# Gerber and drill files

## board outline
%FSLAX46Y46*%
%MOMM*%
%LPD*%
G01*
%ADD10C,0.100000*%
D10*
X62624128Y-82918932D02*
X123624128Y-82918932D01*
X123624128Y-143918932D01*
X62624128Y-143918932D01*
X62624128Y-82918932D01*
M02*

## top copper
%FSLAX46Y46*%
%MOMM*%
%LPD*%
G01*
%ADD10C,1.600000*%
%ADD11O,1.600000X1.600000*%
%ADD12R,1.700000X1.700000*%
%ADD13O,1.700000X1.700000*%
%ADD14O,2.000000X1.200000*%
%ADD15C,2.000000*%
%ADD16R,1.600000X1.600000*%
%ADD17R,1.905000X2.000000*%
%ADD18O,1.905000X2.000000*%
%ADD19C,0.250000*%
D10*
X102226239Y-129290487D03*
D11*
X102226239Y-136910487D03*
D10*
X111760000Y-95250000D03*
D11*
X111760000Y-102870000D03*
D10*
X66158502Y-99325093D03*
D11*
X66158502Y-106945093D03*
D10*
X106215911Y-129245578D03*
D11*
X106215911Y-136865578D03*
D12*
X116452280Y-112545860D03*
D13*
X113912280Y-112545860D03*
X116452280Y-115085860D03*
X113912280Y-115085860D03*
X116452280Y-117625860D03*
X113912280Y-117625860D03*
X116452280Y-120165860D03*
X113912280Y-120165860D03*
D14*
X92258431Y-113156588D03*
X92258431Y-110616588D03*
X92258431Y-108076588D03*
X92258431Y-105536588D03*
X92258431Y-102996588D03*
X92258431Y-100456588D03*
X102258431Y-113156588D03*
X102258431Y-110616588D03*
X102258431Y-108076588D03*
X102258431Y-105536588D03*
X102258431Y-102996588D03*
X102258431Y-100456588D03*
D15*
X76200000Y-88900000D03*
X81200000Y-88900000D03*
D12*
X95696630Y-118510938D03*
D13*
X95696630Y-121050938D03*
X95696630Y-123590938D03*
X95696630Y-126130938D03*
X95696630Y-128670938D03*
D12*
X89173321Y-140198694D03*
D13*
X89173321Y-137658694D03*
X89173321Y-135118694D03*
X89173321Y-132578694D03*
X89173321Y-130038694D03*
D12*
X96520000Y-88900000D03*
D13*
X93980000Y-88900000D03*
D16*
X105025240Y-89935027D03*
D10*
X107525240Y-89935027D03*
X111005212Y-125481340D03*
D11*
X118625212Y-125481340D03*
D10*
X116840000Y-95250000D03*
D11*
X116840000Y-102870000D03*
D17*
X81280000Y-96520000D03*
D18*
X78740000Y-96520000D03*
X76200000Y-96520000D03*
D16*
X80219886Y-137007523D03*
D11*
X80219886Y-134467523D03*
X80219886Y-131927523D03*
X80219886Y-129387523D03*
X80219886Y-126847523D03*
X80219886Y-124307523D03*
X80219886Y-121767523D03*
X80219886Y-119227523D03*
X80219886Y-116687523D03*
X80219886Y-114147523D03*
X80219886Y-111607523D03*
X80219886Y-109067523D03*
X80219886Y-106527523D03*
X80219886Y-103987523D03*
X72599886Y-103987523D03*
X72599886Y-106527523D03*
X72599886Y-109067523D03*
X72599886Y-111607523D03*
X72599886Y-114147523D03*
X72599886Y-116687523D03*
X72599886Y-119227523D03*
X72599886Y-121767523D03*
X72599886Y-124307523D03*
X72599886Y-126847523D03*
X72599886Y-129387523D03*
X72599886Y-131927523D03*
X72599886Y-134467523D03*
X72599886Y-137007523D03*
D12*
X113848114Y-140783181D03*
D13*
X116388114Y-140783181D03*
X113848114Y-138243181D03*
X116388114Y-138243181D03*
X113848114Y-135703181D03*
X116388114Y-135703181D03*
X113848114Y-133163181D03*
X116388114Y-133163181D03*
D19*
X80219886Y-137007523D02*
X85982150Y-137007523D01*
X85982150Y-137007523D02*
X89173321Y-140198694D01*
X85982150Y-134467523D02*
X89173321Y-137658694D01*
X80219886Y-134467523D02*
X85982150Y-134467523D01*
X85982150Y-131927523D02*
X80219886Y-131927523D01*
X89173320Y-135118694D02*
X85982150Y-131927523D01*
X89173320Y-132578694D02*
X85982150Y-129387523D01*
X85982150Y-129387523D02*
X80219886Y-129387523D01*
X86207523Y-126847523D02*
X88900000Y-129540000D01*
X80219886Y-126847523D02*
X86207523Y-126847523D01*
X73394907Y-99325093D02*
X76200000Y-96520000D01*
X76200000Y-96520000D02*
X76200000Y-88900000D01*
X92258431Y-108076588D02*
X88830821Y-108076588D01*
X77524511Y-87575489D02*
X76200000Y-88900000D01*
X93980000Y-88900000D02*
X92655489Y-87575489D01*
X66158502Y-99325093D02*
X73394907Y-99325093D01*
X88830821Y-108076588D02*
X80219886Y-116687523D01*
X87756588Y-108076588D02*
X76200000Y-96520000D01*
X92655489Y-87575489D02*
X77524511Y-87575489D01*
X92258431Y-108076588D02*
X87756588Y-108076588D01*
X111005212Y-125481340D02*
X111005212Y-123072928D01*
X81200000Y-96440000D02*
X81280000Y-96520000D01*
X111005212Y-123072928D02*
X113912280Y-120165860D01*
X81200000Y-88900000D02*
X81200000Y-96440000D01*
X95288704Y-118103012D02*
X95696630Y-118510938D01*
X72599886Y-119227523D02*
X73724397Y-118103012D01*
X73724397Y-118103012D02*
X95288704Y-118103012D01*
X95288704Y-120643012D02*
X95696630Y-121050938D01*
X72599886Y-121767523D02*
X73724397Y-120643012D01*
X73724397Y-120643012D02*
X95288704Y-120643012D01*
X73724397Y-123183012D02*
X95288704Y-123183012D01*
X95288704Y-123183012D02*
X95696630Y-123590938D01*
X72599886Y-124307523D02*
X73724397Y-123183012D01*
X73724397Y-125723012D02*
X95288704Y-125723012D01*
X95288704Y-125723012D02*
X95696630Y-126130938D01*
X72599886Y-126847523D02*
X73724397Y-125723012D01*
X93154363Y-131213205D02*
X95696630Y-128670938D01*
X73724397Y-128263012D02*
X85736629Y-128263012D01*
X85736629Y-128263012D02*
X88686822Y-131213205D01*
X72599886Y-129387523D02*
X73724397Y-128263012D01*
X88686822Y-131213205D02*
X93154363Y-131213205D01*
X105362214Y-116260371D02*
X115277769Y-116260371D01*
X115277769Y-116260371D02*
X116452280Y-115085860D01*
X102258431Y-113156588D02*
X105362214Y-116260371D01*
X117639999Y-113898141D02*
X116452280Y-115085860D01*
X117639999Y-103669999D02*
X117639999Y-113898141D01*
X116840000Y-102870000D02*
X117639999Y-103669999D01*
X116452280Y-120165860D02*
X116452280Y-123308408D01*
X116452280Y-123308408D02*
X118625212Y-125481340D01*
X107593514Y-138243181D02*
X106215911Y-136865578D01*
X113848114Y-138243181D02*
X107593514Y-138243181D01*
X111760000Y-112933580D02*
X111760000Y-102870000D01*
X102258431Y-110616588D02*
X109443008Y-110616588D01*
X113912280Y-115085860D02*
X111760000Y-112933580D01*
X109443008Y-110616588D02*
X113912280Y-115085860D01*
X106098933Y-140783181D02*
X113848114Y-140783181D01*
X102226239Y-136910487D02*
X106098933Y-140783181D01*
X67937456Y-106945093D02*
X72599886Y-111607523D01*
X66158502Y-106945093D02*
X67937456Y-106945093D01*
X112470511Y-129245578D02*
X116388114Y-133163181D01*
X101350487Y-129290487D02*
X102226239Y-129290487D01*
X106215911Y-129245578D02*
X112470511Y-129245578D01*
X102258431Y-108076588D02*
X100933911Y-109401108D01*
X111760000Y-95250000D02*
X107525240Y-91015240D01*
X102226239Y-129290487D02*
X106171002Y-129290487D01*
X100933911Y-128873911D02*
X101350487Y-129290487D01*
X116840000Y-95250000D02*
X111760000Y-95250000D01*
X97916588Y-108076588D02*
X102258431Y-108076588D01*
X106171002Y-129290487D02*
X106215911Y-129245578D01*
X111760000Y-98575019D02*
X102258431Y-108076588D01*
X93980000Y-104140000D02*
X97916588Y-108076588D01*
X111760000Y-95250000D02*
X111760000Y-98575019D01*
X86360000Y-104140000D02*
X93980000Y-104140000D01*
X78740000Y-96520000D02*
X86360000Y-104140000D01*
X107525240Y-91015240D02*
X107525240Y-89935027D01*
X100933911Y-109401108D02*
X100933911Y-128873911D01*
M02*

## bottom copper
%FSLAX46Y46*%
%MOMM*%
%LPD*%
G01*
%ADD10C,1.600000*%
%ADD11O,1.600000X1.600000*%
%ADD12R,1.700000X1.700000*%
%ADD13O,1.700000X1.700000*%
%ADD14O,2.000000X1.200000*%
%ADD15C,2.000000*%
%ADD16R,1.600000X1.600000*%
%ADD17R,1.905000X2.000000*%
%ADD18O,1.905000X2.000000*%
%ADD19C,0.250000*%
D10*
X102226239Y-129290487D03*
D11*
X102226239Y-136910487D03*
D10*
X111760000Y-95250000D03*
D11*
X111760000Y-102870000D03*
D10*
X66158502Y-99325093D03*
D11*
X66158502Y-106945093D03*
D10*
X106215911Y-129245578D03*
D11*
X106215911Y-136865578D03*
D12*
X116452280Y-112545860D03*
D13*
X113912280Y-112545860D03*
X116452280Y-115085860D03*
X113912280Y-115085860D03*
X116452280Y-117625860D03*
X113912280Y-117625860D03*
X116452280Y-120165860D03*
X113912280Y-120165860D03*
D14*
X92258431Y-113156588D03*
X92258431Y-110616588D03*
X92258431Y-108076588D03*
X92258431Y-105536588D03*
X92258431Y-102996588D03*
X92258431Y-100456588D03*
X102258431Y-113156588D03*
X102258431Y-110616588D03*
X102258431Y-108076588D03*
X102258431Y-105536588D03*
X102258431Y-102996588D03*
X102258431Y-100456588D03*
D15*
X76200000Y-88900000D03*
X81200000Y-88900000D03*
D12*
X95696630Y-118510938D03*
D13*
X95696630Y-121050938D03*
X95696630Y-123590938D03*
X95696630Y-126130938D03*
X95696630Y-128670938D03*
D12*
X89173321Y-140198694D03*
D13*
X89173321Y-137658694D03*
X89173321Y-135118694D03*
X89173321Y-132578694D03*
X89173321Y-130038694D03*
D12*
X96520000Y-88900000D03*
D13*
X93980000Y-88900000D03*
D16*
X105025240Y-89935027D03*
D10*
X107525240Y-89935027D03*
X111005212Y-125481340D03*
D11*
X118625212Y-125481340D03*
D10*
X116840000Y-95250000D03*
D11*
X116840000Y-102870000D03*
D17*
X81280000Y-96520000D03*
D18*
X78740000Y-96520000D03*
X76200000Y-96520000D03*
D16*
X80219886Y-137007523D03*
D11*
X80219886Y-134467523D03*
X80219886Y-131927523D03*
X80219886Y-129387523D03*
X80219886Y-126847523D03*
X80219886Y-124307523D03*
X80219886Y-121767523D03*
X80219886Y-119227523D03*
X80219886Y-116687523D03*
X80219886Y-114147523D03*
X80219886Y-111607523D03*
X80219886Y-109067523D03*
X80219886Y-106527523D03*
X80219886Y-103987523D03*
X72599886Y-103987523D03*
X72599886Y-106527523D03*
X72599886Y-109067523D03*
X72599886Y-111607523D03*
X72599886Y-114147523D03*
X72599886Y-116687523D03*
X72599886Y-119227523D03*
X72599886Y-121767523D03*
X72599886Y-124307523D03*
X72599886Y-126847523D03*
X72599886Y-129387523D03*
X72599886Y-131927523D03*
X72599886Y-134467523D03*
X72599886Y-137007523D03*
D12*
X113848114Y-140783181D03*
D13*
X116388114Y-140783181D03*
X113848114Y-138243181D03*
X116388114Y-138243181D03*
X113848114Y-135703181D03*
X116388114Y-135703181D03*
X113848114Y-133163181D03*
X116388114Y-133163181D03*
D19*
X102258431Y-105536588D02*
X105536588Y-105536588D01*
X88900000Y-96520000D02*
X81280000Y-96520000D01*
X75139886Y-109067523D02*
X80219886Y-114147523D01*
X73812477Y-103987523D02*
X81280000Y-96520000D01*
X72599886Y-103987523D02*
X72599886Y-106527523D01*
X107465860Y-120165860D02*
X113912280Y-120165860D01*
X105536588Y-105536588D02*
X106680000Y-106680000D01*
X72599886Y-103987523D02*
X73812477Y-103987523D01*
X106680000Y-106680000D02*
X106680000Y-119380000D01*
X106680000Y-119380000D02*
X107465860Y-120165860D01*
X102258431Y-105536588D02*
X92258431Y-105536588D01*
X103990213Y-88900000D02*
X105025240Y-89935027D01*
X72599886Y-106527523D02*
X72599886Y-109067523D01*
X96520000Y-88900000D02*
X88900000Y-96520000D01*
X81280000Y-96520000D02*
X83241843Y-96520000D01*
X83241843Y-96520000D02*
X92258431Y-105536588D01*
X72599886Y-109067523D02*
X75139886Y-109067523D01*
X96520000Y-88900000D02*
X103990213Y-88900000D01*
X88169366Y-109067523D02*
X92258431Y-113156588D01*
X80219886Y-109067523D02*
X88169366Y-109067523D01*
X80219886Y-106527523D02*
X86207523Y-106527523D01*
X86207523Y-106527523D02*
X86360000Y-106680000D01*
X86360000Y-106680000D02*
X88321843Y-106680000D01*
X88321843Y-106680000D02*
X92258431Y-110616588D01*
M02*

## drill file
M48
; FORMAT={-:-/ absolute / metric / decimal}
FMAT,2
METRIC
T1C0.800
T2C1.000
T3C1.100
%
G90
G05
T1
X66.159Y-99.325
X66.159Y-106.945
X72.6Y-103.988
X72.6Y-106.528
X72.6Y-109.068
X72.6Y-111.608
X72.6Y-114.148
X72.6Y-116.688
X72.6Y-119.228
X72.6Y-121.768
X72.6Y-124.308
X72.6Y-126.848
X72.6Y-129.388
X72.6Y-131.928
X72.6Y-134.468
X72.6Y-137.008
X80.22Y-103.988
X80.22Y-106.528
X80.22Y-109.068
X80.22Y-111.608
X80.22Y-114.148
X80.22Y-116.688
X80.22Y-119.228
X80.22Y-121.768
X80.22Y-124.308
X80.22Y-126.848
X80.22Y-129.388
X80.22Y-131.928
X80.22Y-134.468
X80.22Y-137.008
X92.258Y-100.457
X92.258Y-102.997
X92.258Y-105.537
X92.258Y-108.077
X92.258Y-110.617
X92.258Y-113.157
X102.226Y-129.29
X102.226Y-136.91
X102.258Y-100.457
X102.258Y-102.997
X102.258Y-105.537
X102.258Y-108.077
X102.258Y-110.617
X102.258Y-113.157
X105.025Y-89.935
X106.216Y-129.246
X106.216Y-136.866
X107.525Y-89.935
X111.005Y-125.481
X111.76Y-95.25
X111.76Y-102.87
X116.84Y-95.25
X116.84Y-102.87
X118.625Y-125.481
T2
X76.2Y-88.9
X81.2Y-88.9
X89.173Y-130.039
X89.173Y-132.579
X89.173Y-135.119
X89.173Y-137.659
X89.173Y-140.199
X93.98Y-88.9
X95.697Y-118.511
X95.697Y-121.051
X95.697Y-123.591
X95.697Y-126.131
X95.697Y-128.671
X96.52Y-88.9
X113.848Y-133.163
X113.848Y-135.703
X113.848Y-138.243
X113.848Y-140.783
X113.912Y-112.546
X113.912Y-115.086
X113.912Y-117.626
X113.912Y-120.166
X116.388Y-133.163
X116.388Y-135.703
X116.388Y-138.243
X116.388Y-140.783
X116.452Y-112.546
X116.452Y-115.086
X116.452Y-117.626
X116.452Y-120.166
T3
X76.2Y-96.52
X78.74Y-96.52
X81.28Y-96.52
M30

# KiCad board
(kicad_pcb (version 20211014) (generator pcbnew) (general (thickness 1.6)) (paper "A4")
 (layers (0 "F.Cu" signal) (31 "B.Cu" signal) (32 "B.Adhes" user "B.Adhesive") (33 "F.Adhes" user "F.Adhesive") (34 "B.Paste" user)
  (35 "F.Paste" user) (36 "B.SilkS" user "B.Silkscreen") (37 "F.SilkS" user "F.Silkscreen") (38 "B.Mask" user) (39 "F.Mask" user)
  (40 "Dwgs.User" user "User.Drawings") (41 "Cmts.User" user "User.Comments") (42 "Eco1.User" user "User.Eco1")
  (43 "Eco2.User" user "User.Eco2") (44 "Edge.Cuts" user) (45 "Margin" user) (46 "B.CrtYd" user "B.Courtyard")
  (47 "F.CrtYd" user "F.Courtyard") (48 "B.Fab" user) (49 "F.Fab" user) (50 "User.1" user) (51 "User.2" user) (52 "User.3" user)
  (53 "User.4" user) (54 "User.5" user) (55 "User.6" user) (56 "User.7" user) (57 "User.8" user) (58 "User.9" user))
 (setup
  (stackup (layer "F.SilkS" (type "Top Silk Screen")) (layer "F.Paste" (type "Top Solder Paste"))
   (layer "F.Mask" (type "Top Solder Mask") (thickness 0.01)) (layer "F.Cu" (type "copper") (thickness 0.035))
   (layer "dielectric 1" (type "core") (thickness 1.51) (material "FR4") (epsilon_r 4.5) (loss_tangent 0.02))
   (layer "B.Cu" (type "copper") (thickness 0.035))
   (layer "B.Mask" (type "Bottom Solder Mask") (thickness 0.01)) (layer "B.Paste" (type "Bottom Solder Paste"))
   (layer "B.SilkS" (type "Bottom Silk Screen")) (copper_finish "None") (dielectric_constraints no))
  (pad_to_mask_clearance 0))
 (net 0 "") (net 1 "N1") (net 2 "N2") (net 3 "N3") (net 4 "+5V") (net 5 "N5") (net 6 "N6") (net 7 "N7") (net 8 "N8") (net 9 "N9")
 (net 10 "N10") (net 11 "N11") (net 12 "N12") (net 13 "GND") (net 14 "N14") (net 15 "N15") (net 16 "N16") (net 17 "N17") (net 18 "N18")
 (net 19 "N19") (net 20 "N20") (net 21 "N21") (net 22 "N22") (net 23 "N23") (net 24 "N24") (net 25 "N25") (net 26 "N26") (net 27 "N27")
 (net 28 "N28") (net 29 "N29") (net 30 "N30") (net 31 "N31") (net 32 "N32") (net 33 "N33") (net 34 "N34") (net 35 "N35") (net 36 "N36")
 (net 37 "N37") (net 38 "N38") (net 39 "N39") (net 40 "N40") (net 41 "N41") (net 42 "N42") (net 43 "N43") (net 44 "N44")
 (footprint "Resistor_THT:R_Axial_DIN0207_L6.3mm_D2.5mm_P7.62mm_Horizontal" (layer "F.Cu") (at 102.226239 129.290487 -90)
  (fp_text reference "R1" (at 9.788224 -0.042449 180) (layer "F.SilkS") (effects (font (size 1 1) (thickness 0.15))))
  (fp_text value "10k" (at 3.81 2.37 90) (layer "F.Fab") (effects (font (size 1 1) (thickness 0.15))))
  (pad "1" thru_hole circle (at 0 0 270) (size 1.6 1.6) (drill 0.8) (layers *.Cu *.Mask) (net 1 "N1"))
  (pad "2" thru_hole oval (at 7.62 0 270) (size 1.6 1.6) (drill 0.8) (layers *.Cu *.Mask) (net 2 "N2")))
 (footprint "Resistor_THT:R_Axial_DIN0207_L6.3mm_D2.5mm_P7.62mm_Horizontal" (layer "F.Cu") (at 111.76 95.25 -90)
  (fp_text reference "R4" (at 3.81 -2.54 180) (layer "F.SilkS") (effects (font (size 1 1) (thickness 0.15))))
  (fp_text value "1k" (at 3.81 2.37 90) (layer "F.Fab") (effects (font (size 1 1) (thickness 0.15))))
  (pad "1" thru_hole circle (at 0 0 270) (size 1.6 1.6) (drill 0.8) (layers *.Cu *.Mask) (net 1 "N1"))
  (pad "2" thru_hole oval (at 7.62 0 270) (size 1.6 1.6) (drill 0.8) (layers *.Cu *.Mask) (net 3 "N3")))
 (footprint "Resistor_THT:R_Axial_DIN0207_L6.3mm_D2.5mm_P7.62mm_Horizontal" (layer "F.Cu") (at 66.158502 99.325093 -90)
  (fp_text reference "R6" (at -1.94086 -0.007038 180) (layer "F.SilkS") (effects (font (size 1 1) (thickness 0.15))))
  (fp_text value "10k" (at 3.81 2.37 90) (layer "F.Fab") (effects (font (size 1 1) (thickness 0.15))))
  (pad "1" thru_hole circle (at 0 0 270) (size 1.6 1.6) (drill 0.8) (layers *.Cu *.Mask) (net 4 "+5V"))
  (pad "2" thru_hole oval (at 7.62 0 270) (size 1.6 1.6) (drill 0.8) (layers *.Cu *.Mask) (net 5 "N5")))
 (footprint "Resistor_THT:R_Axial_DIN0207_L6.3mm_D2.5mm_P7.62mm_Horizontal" (layer "F.Cu") (at 106.215911 129.245578 -90)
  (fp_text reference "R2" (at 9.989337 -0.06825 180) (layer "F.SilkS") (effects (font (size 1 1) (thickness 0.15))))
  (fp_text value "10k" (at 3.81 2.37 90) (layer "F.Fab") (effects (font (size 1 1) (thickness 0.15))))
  (pad "1" thru_hole circle (at 0 0 270) (size 1.6 1.6) (drill 0.8) (layers *.Cu *.Mask) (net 1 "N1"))
  (pad "2" thru_hole oval (at 7.62 0 270) (size 1.6 1.6) (drill 0.8) (layers *.Cu *.Mask) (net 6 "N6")))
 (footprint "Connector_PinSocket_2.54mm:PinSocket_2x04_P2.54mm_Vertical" (layer "F.Cu") (at 116.45228 112.54586)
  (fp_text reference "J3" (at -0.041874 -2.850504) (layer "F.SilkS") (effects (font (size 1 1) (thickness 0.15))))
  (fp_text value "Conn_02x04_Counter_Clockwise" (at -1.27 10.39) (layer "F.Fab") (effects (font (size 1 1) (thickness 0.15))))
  (pad "1" thru_hole rect (at 0 0) (size 1.7 1.7) (drill 1) (layers *.Cu *.Mask) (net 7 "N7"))
  (pad "2" thru_hole oval (at -2.54 0) (size 1.7 1.7) (drill 1) (layers *.Cu *.Mask) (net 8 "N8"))
  (pad "3" thru_hole oval (at 0 2.54) (size 1.7 1.7) (drill 1) (layers *.Cu *.Mask) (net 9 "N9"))
  (pad "4" thru_hole oval (at -2.54 2.54) (size 1.7 1.7) (drill 1) (layers *.Cu *.Mask) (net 3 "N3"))
  (pad "5" thru_hole oval (at 0 5.08) (size 1.7 1.7) (drill 1) (layers *.Cu *.Mask) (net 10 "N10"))
  (pad "6" thru_hole oval (at -2.54 5.08) (size 1.7 1.7) (drill 1) (layers *.Cu *.Mask) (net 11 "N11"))
  (pad "7" thru_hole oval (at 0 7.62) (size 1.7 1.7) (drill 1) (layers *.Cu *.Mask) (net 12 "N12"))
  (pad "8" thru_hole oval (at -2.54 7.62) (size 1.7 1.7) (drill 1) (layers *.Cu *.Mask) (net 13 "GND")))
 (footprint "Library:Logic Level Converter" (layer "F.Cu") (at 97.258431 106.806588 90)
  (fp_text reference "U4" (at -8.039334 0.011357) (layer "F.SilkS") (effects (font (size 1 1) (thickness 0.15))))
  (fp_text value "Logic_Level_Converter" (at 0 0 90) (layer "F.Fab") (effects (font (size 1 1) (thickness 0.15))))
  (pad "1" thru_hole oval (at -6.35 -5 90) (size 1.2 2) (drill 0.8) (layers *.Cu *.Mask) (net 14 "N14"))
  (pad "2" thru_hole oval (at -3.81 -5 90) (size 1.2 2) (drill 0.8) (layers *.Cu *.Mask) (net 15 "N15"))
  (pad "3" thru_hole oval (at -1.27 -5 90) (size 1.2 2) (drill 0.8) (layers *.Cu *.Mask) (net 4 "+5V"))
  (pad "4" thru_hole oval (at 1.27 -5 90) (size 1.2 2) (drill 0.8) (layers *.Cu *.Mask) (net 13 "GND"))
  (pad "5" thru_hole oval (at 3.81 -5 90) (size 1.2 2) (drill 0.8) (layers *.Cu *.Mask) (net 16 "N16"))
  (pad "6" thru_hole oval (at 6.35 -5 90) (size 1.2 2) (drill 0.8) (layers *.Cu *.Mask) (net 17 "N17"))
  (pad "7" thru_hole oval (at -6.35 5 90) (size 1.2 2) (drill 0.8) (layers *.Cu *.Mask) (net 9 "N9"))
  (pad "8" thru_hole oval (at -3.81 5 90) (size 1.2 2) (drill 0.8) (layers *.Cu *.Mask) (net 3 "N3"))
  (pad "9" thru_hole oval (at -1.27 5 90) (size 1.2 2) (drill 0.8) (layers *.Cu *.Mask) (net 1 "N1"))
  (pad "10" thru_hole oval (at 1.27 5 90) (size 1.2 2) (drill 0.8) (layers *.Cu *.Mask) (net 13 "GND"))
  (pad "11" thru_hole oval (at 3.81 5 90) (size 1.2 2) (drill 0.8) (layers *.Cu *.Mask) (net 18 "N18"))
  (pad "12" thru_hole oval (at 6.35 5 90) (size 1.2 2) (drill 0.8) (layers *.Cu *.Mask) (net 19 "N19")))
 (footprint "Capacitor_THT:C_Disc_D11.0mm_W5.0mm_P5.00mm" (layer "F.Cu") (at 76.2 88.9)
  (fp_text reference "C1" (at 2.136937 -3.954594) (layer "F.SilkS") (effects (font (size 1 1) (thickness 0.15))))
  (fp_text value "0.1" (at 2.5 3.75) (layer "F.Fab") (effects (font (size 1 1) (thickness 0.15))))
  (pad "1" thru_hole circle (at 0 0) (size 2 2) (drill 1) (layers *.Cu *.Mask) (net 4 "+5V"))
  (pad "2" thru_hole circle (at 5 0) (size 2 2) (drill 1) (layers *.Cu *.Mask) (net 13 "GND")))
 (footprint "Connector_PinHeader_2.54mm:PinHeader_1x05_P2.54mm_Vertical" (layer "F.Cu") (at 95.69663 118.510938)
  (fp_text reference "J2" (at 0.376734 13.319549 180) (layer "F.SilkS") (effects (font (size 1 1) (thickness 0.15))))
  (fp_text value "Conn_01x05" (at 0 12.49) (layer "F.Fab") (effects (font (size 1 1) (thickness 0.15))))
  (pad "1" thru_hole rect (at 0 0) (size 1.7 1.7) (drill 1) (layers *.Cu *.Mask) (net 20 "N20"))
  (pad "2" thru_hole oval (at 0 2.54) (size 1.7 1.7) (drill 1) (layers *.Cu *.Mask) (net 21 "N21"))
  (pad "3" thru_hole oval (at 0 5.08) (size 1.7 1.7) (drill 1) (layers *.Cu *.Mask) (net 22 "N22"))
  (pad "4" thru_hole oval (at 0 7.62) (size 1.7 1.7) (drill 1) (layers *.Cu *.Mask) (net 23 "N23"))
  (pad "5" thru_hole oval (at 0 10.16) (size 1.7 1.7) (drill 1) (layers *.Cu *.Mask) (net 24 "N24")))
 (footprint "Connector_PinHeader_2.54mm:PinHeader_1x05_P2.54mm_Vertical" (layer "F.Cu") (at 89.173321 140.198694 180)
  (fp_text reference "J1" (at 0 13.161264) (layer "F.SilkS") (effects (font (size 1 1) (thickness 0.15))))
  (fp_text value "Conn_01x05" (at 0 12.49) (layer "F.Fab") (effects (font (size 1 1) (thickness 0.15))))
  (pad "1" thru_hole rect (at 0 0 180) (size 1.7 1.7) (drill 1) (layers *.Cu *.Mask) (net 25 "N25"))
  (pad "2" thru_hole oval (at 0 2.54 180) (size 1.7 1.7) (drill 1) (layers *.Cu *.Mask) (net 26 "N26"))
  (pad "3" thru_hole oval (at 0 5.08 180) (size 1.7 1.7) (drill 1) (layers *.Cu *.Mask) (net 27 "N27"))
  (pad "4" thru_hole oval (at 0 7.62 180) (size 1.7 1.7) (drill 1) (layers *.Cu *.Mask) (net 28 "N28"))
  (pad "5" thru_hole oval (at 0 10.16 180) (size 1.7 1.7) (drill 1) (layers *.Cu *.Mask) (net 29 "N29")))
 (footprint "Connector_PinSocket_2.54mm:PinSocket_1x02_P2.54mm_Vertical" (layer "F.Cu") (at 96.52 88.9 -90)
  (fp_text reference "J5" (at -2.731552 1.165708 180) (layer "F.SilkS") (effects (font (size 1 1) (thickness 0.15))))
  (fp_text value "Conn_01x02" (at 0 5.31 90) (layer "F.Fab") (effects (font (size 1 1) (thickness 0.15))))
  (pad "1" thru_hole rect (at 0 0 270) (size 1.7 1.7) (drill 1) (layers *.Cu *.Mask) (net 13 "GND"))
  (pad "2" thru_hole oval (at 0 2.54 270) (size 1.7 1.7) (drill 1) (layers *.Cu *.Mask) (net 4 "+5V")))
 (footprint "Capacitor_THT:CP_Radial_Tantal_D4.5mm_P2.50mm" (layer "F.Cu") (at 105.02524 89.935027)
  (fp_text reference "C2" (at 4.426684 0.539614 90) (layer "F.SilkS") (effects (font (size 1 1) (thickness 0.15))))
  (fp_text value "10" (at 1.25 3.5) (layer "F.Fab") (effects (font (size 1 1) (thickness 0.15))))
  (pad "1" thru_hole rect (at 0 0) (size 1.6 1.6) (drill 0.8) (layers *.Cu *.Mask) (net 13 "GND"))
  (pad "2" thru_hole circle (at 2.5 0) (size 1.6 1.6) (drill 0.8) (layers *.Cu *.Mask) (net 1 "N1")))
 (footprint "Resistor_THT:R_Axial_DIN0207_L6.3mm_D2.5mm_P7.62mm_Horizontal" (layer "F.Cu") (at 111.005212 125.48134)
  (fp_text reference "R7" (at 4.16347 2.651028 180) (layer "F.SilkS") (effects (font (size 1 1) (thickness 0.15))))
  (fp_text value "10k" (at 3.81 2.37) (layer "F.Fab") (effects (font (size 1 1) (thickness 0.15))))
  (pad "1" thru_hole circle (at 0 0) (size 1.6 1.6) (drill 0.8) (layers *.Cu *.Mask) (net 13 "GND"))
  (pad "2" thru_hole oval (at 7.62 0) (size 1.6 1.6) (drill 0.8) (layers *.Cu *.Mask) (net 12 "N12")))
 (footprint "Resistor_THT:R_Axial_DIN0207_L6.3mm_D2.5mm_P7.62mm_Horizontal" (layer "F.Cu") (at 116.84 95.25 -90)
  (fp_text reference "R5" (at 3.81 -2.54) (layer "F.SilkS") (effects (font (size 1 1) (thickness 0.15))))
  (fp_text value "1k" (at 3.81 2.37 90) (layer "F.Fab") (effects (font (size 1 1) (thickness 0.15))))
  (pad "1" thru_hole circle (at 0 0 270) (size 1.6 1.6) (drill 0.8) (layers *.Cu *.Mask) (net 1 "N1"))
  (pad "2" thru_hole oval (at 7.62 0 270) (size 1.6 1.6) (drill 0.8) (layers *.Cu *.Mask) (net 9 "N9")))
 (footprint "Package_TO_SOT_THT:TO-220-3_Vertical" (layer "F.Cu") (at 81.28 96.52 180)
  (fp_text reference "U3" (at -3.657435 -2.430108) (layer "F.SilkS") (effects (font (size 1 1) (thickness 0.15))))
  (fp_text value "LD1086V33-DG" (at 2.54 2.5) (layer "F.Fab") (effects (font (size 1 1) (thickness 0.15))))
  (pad "1" thru_hole rect (at 0 0 180) (size 1.905 2) (drill 1.1) (layers *.Cu *.Mask) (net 13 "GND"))
  (pad "2" thru_hole oval (at 2.54 0 180) (size 1.905 2) (drill 1.1) (layers *.Cu *.Mask) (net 1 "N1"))
  (pad "3" thru_hole oval (at 5.08 0 180) (size 1.905 2) (drill 1.1) (layers *.Cu *.Mask) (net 4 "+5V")))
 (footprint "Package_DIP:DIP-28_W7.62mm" (layer "F.Cu") (at 80.219886 137.007523 180)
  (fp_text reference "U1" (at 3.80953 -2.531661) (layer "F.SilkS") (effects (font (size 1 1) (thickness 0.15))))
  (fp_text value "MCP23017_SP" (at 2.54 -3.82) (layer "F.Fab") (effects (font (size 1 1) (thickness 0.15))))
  (pad "1" thru_hole rect (at 0 0 180) (size 1.6 1.6) (drill 0.8) (layers *.Cu *.Mask) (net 25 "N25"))
  (pad "2" thru_hole oval (at 0 2.54 180) (size 1.6 1.6) (drill 0.8) (layers *.Cu *.Mask) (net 26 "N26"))
  (pad "3" thru_hole oval (at 0 5.08 180) (size 1.6 1.6) (drill 0.8) (layers *.Cu *.Mask) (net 27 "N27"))
  (pad "4" thru_hole oval (at 0 7.62 180) (size 1.6 1.6) (drill 0.8) (layers *.Cu *.Mask) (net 28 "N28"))
  (pad "5" thru_hole oval (at 0 10.16 180) (size 1.6 1.6) (drill 0.8) (layers *.Cu *.Mask) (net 29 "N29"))
  (pad "6" thru_hole oval (at 0 12.7 180) (size 1.6 1.6) (drill 0.8) (layers *.Cu *.Mask) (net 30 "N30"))
  (pad "7" thru_hole oval (at 0 15.24 180) (size 1.6 1.6) (drill 0.8) (layers *.Cu *.Mask) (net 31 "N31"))
  (pad "8" thru_hole oval (at 0 17.78 180) (size 1.6 1.6) (drill 0.8) (layers *.Cu *.Mask) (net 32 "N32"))
  (pad "9" thru_hole oval (at 0 20.32 180) (size 1.6 1.6) (drill 0.8) (layers *.Cu *.Mask) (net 4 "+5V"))
  (pad "10" thru_hole oval (at 0 22.86 180) (size 1.6 1.6) (drill 0.8) (layers *.Cu *.Mask) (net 13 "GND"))
  (pad "11" thru_hole oval (at 0 25.4 180) (size 1.6 1.6) (drill 0.8) (layers *.Cu *.Mask) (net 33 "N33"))
  (pad "12" thru_hole oval (at 0 27.94 180) (size 1.6 1.6) (drill 0.8) (layers *.Cu *.Mask) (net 14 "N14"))
  (pad "13" thru_hole oval (at 0 30.48 180) (size 1.6 1.6) (drill 0.8) (layers *.Cu *.Mask) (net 15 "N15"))
  (pad "14" thru_hole oval (at 0 33.02 180) (size 1.6 1.6) (drill 0.8) (layers *.Cu *.Mask) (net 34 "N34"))
  (pad "15" thru_hole oval (at 7.62 33.02 180) (size 1.6 1.6) (drill 0.8) (layers *.Cu *.Mask) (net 13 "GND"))
  (pad "16" thru_hole oval (at 7.62 30.48 180) (size 1.6 1.6) (drill 0.8) (layers *.Cu *.Mask) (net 13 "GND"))
  (pad "17" thru_hole oval (at 7.62 27.94 180) (size 1.6 1.6) (drill 0.8) (layers *.Cu *.Mask) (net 13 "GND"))
  (pad "18" thru_hole oval (at 7.62 25.4 180) (size 1.6 1.6) (drill 0.8) (layers *.Cu *.Mask) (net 5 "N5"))
  (pad "19" thru_hole oval (at 7.62 22.86 180) (size 1.6 1.6) (drill 0.8) (layers *.Cu *.Mask) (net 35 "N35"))
  (pad "20" thru_hole oval (at 7.62 20.32 180) (size 1.6 1.6) (drill 0.8) (layers *.Cu *.Mask) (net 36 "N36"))
  (pad "21" thru_hole oval (at 7.62 17.78 180) (size 1.6 1.6) (drill 0.8) (layers *.Cu *.Mask) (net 20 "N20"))
  (pad "22" thru_hole oval (at 7.62 15.24 180) (size 1.6 1.6) (drill 0.8) (layers *.Cu *.Mask) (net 21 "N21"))
  (pad "23" thru_hole oval (at 7.62 12.7 180) (size 1.6 1.6) (drill 0.8) (layers *.Cu *.Mask) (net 22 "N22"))
  (pad "24" thru_hole oval (at 7.62 10.16 180) (size 1.6 1.6) (drill 0.8) (layers *.Cu *.Mask) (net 23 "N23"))
  (pad "25" thru_hole oval (at 7.62 7.62 180) (size 1.6 1.6) (drill 0.8) (layers *.Cu *.Mask) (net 24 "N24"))
  (pad "26" thru_hole oval (at 7.62 5.08 180) (size 1.6 1.6) (drill 0.8) (layers *.Cu *.Mask) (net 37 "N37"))
  (pad "27" thru_hole oval (at 7.62 2.54 180) (size 1.6 1.6) (drill 0.8) (layers *.Cu *.Mask) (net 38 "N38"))
  (pad "28" thru_hole oval (at 7.62 0 180) (size 1.6 1.6) (drill 0.8) (layers *.Cu *.Mask) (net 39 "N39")))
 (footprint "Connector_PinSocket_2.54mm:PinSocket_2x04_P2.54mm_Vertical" (layer "F.Cu") (at 113.848114 140.783181 180)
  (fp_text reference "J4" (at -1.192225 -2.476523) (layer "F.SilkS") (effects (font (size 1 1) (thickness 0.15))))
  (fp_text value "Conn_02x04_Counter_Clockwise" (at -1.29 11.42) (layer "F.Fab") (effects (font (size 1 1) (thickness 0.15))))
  (pad "1" thru_hole rect (at 0 0 180) (size 1.7 1.7) (drill 1) (layers *.Cu *.Mask) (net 2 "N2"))
  (pad "2" thru_hole oval (at -2.54 0 180) (size 1.7 1.7) (drill 1) (layers *.Cu *.Mask) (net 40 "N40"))
  (pad "3" thru_hole oval (at 0 2.54 180) (size 1.7 1.7) (drill 1) (layers *.Cu *.Mask) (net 6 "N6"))
  (pad "4" thru_hole oval (at -2.54 2.54 180) (size 1.7 1.7) (drill 1) (layers *.Cu *.Mask) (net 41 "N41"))
  (pad "5" thru_hole oval (at 0 5.08 180) (size 1.7 1.7) (drill 1) (layers *.Cu *.Mask) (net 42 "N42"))
  (pad "6" thru_hole oval (at -2.54 5.08 180) (size 1.7 1.7) (drill 1) (layers *.Cu *.Mask) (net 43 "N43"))
  (pad "7" thru_hole oval (at 0 7.62 180) (size 1.7 1.7) (drill 1) (layers *.Cu *.Mask) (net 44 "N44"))
  (pad "8" thru_hole oval (at -2.54 7.62 180) (size 1.7 1.7) (drill 1) (layers *.Cu *.Mask) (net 1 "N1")))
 (gr_rect (start 96.52 81.28) (end 96.52 81.28) (layer "Edge.Cuts") (width 0.1) (fill none))
 (gr_rect (start 62.624128 82.918932) (end 123.624128 143.918932) (layer "Edge.Cuts") (width 0.1) (fill none))
 (segment (start 80.219886 137.007523) (end 85.98215 137.007523) (width 0.25) (layer "F.Cu") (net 25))
 (segment (start 85.98215 137.007523) (end 89.173321 140.198694) (width 0.25) (layer "F.Cu") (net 25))
 (segment (start 85.98215 134.467523) (end 89.173321 137.658694) (width 0.25) (layer "F.Cu") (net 26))
 (segment (start 80.219886 134.467523) (end 85.98215 134.467523) (width 0.25) (layer "F.Cu") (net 26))
 (segment (start 85.98215 131.927523) (end 80.219886 131.927523) (width 0.25) (layer "F.Cu") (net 27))
 (segment (start 89.17332 135.118694) (end 85.98215 131.927523) (width 0.25) (layer "F.Cu") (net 27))
 (segment (start 89.17332 132.578694) (end 85.98215 129.387523) (width 0.25) (layer "F.Cu") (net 28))
 (segment (start 85.98215 129.387523) (end 80.219886 129.387523) (width 0.25) (layer "F.Cu") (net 28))
 (segment (start 86.207523 126.847523) (end 88.9 129.54) (width 0.25) (layer "F.Cu") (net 29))
 (segment (start 80.219886 126.847523) (end 86.207523 126.847523) (width 0.25) (layer "F.Cu") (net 29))
 (segment (start 73.394907 99.325093) (end 76.2 96.52) (width 0.25) (layer "F.Cu") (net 4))
 (segment (start 76.2 96.52) (end 76.2 88.9) (width 0.25) (layer "F.Cu") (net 4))
 (segment (start 92.258431 108.076588) (end 88.830821 108.076588) (width 0.25) (layer "F.Cu") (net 4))
 (segment (start 77.524511 87.575489) (end 76.2 88.9) (width 0.25) (layer "F.Cu") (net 4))
 (segment (start 93.98 88.9) (end 92.655489 87.575489) (width 0.25) (layer "F.Cu") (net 4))
 (segment (start 66.158502 99.325093) (end 73.394907 99.325093) (width 0.25) (layer "F.Cu") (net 4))
 (segment (start 88.830821 108.076588) (end 80.219886 116.687523) (width 0.25) (layer "F.Cu") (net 4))
 (segment (start 87.756588 108.076588) (end 76.2 96.52) (width 0.25) (layer "F.Cu") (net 4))
 (segment (start 92.655489 87.575489) (end 77.524511 87.575489) (width 0.25) (layer "F.Cu") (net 4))
 (segment (start 92.258431 108.076588) (end 87.756588 108.076588) (width 0.25) (layer "F.Cu") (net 4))
 (segment (start 111.005212 125.48134) (end 111.005212 123.072928) (width 0.25) (layer "F.Cu") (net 13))
 (segment (start 81.2 96.44) (end 81.28 96.52) (width 0.25) (layer "F.Cu") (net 13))
 (segment (start 111.005212 123.072928) (end 113.91228 120.16586) (width 0.25) (layer "F.Cu") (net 13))
 (segment (start 81.2 88.9) (end 81.2 96.44) (width 0.25) (layer "F.Cu") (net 13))
 (segment (start 102.258431 105.536588) (end 105.536588 105.536588) (width 0.25) (layer "B.Cu") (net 13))
 (segment (start 88.9 96.52) (end 81.28 96.52) (width 0.25) (layer "B.Cu") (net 13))
 (segment (start 75.139886 109.067523) (end 80.219886 114.147523) (width 0.25) (layer "B.Cu") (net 13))
 (segment (start 73.812477 103.987523) (end 81.28 96.52) (width 0.25) (layer "B.Cu") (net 13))
 (segment (start 72.599886 103.987523) (end 72.599886 106.527523) (width 0.25) (layer "B.Cu") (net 13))
 (segment (start 107.46586 120.16586) (end 113.91228 120.16586) (width 0.25) (layer "B.Cu") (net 13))
 (segment (start 105.536588 105.536588) (end 106.68 106.68) (width 0.25) (layer "B.Cu") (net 13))
 (segment (start 72.599886 103.987523) (end 73.812477 103.987523) (width 0.25) (layer "B.Cu") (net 13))
 (segment (start 106.68 106.68) (end 106.68 119.38) (width 0.25) (layer "B.Cu") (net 13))
 (segment (start 106.68 119.38) (end 107.46586 120.16586) (width 0.25) (layer "B.Cu") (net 13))
 (segment (start 102.258431 105.536588) (end 92.258431 105.536588) (width 0.25) (layer "B.Cu") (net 13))
 (segment (start 103.990213 88.9) (end 105.02524 89.935027) (width 0.25) (layer "B.Cu") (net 13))
 (segment (start 72.599886 106.527523) (end 72.599886 109.067523) (width 0.25) (layer "B.Cu") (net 13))
 (segment (start 96.52 88.9) (end 88.9 96.52) (width 0.25) (layer "B.Cu") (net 13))
 (segment (start 81.28 96.52) (end 83.241843 96.52) (width 0.25) (layer "B.Cu") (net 13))
 (segment (start 83.241843 96.52) (end 92.258431 105.536588) (width 0.25) (layer "B.Cu") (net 13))
 (segment (start 72.599886 109.067523) (end 75.139886 109.067523) (width 0.25) (layer "B.Cu") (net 13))
 (segment (start 96.52 88.9) (end 103.990213 88.9) (width 0.25) (layer "B.Cu") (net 13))
 (segment (start 88.169366 109.067523) (end 92.258431 113.156588) (width 0.25) (layer "B.Cu") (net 14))
 (segment (start 80.219886 109.067523) (end 88.169366 109.067523) (width 0.25) (layer "B.Cu") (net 14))
 (segment (start 95.288704 118.103012) (end 95.69663 118.510938) (width 0.25) (layer "F.Cu") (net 20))
 (segment (start 72.599886 119.227523) (end 73.724397 118.103012) (width 0.25) (layer "F.Cu") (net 20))
 (segment (start 73.724397 118.103012) (end 95.288704 118.103012) (width 0.25) (layer "F.Cu") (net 20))
 (segment (start 95.288704 120.643012) (end 95.69663 121.050938) (width 0.25) (layer "F.Cu") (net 21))
 (segment (start 72.599886 121.767523) (end 73.724397 120.643012) (width 0.25) (layer "F.Cu") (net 21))
 (segment (start 73.724397 120.643012) (end 95.288704 120.643012) (width 0.25) (layer "F.Cu") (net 21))
 (segment (start 73.724397 123.183012) (end 95.288704 123.183012) (width 0.25) (layer "F.Cu") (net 22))
 (segment (start 95.288704 123.183012) (end 95.69663 123.590938) (width 0.25) (layer "F.Cu") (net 22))
 (segment (start 72.599886 124.307523) (end 73.724397 123.183012) (width 0.25) (layer "F.Cu") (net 22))
 (segment (start 73.724397 125.723012) (end 95.288704 125.723012) (width 0.25) (layer "F.Cu") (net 23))
 (segment (start 95.288704 125.723012) (end 95.69663 126.130938) (width 0.25) (layer "F.Cu") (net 23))
 (segment (start 72.599886 126.847523) (end 73.724397 125.723012) (width 0.25) (layer "F.Cu") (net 23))
 (segment (start 93.154363 131.213205) (end 95.69663 128.670938) (width 0.25) (layer "F.Cu") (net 24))
 (segment (start 73.724397 128.263012) (end 85.736629 128.263012) (width 0.25) (layer "F.Cu") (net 24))
 (segment (start 85.736629 128.263012) (end 88.686822 131.213205) (width 0.25) (layer "F.Cu") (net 24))
 (segment (start 72.599886 129.387523) (end 73.724397 128.263012) (width 0.25) (layer "F.Cu") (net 24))
 (segment (start 88.686822 131.213205) (end 93.154363 131.213205) (width 0.25) (layer "F.Cu") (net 24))
 (segment (start 105.362214 116.260371) (end 115.277769 116.260371) (width 0.25) (layer "F.Cu") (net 9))
 (segment (start 115.277769 116.260371) (end 116.45228 115.08586) (width 0.25) (layer "F.Cu") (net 9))
 (segment (start 102.258431 113.156588) (end 105.362214 116.260371) (width 0.25) (layer "F.Cu") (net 9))
 (segment (start 117.639999 113.898141) (end 116.45228 115.08586) (width 0.25) (layer "F.Cu") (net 9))
 (segment (start 117.639999 103.669999) (end 117.639999 113.898141) (width 0.25) (layer "F.Cu") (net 9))
 (segment (start 116.84 102.87) (end 117.639999 103.669999) (width 0.25) (layer "F.Cu") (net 9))
 (segment (start 116.45228 120.16586) (end 116.45228 123.308408) (width 0.25) (layer "F.Cu") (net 12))
 (segment (start 116.45228 123.308408) (end 118.625212 125.48134) (width 0.25) (layer "F.Cu") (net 12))
 (segment (start 107.593514 138.243181) (end 106.215911 136.865578) (width 0.25) (layer "F.Cu") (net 6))
 (segment (start 113.848114 138.243181) (end 107.593514 138.243181) (width 0.25) (layer "F.Cu") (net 6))
 (segment (start 111.76 112.93358) (end 111.76 102.87) (width 0.25) (layer "F.Cu") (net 3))
 (segment (start 102.258431 110.616588) (end 109.443008 110.616588) (width 0.25) (layer "F.Cu") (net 3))
 (segment (start 113.91228 115.08586) (end 111.76 112.93358) (width 0.25) (layer "F.Cu") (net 3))
 (segment (start 109.443008 110.616588) (end 113.91228 115.08586) (width 0.25) (layer "F.Cu") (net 3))
 (segment (start 106.098933 140.783181) (end 113.848114 140.783181) (width 0.25) (layer "F.Cu") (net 2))
 (segment (start 102.226239 136.910487) (end 106.098933 140.783181) (width 0.25) (layer "F.Cu") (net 2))
 (segment (start 67.937456 106.945093) (end 72.599886 111.607523) (width 0.25) (layer "F.Cu") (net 5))
 (segment (start 66.158502 106.945093) (end 67.937456 106.945093) (width 0.25) (layer "F.Cu") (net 5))
 (segment (start 80.219886 106.527523) (end 86.207523 106.527523) (width 0.25) (layer "B.Cu") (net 15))
 (segment (start 86.207523 106.527523) (end 86.36 106.68) (width 0.25) (layer "B.Cu") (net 15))
 (segment (start 86.36 106.68) (end 88.321843 106.68) (width 0.25) (layer "B.Cu") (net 15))
 (segment (start 88.321843 106.68) (end 92.258431 110.616588) (width 0.25) (layer "B.Cu") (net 15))
 (segment (start 112.470511 129.245578) (end 116.388114 133.163181) (width 0.25) (layer "F.Cu") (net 1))
 (segment (start 101.350487 129.290487) (end 102.226239 129.290487) (width 0.25) (layer "F.Cu") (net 1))
 (segment (start 106.215911 129.245578) (end 112.470511 129.245578) (width 0.25) (layer "F.Cu") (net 1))
 (segment (start 102.258431 108.076588) (end 100.933911 109.401108) (width 0.25) (layer "F.Cu") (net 1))
 (segment (start 111.76 95.25) (end 107.52524 91.01524) (width 0.25) (layer "F.Cu") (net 1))
 (segment (start 102.226239 129.290487) (end 106.171002 129.290487) (width 0.25) (layer "F.Cu") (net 1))
 (segment (start 100.933911 128.873911) (end 101.350487 129.290487) (width 0.25) (layer "F.Cu") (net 1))
 (segment (start 116.84 95.25) (end 111.76 95.25) (width 0.25) (layer "F.Cu") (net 1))
 (segment (start 97.916588 108.076588) (end 102.258431 108.076588) (width 0.25) (layer "F.Cu") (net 1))
 (segment (start 106.171002 129.290487) (end 106.215911 129.245578) (width 0.25) (layer "F.Cu") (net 1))
 (segment (start 111.76 98.575019) (end 102.258431 108.076588) (width 0.25) (layer "F.Cu") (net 1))
 (segment (start 93.98 104.14) (end 97.916588 108.076588) (width 0.25) (layer "F.Cu") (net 1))
 (segment (start 111.76 95.25) (end 111.76 98.575019) (width 0.25) (layer "F.Cu") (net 1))
 (segment (start 86.36 104.14) (end 93.98 104.14) (width 0.25) (layer "F.Cu") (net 1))
 (segment (start 78.74 96.52) (end 86.36 104.14) (width 0.25) (layer "F.Cu") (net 1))
 (segment (start 107.52524 91.01524) (end 107.52524 89.935027) (width 0.25) (layer "F.Cu") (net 1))
 (segment (start 100.933911 109.401108) (end 100.933911 128.873911) (width 0.25) (layer "F.Cu") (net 1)))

